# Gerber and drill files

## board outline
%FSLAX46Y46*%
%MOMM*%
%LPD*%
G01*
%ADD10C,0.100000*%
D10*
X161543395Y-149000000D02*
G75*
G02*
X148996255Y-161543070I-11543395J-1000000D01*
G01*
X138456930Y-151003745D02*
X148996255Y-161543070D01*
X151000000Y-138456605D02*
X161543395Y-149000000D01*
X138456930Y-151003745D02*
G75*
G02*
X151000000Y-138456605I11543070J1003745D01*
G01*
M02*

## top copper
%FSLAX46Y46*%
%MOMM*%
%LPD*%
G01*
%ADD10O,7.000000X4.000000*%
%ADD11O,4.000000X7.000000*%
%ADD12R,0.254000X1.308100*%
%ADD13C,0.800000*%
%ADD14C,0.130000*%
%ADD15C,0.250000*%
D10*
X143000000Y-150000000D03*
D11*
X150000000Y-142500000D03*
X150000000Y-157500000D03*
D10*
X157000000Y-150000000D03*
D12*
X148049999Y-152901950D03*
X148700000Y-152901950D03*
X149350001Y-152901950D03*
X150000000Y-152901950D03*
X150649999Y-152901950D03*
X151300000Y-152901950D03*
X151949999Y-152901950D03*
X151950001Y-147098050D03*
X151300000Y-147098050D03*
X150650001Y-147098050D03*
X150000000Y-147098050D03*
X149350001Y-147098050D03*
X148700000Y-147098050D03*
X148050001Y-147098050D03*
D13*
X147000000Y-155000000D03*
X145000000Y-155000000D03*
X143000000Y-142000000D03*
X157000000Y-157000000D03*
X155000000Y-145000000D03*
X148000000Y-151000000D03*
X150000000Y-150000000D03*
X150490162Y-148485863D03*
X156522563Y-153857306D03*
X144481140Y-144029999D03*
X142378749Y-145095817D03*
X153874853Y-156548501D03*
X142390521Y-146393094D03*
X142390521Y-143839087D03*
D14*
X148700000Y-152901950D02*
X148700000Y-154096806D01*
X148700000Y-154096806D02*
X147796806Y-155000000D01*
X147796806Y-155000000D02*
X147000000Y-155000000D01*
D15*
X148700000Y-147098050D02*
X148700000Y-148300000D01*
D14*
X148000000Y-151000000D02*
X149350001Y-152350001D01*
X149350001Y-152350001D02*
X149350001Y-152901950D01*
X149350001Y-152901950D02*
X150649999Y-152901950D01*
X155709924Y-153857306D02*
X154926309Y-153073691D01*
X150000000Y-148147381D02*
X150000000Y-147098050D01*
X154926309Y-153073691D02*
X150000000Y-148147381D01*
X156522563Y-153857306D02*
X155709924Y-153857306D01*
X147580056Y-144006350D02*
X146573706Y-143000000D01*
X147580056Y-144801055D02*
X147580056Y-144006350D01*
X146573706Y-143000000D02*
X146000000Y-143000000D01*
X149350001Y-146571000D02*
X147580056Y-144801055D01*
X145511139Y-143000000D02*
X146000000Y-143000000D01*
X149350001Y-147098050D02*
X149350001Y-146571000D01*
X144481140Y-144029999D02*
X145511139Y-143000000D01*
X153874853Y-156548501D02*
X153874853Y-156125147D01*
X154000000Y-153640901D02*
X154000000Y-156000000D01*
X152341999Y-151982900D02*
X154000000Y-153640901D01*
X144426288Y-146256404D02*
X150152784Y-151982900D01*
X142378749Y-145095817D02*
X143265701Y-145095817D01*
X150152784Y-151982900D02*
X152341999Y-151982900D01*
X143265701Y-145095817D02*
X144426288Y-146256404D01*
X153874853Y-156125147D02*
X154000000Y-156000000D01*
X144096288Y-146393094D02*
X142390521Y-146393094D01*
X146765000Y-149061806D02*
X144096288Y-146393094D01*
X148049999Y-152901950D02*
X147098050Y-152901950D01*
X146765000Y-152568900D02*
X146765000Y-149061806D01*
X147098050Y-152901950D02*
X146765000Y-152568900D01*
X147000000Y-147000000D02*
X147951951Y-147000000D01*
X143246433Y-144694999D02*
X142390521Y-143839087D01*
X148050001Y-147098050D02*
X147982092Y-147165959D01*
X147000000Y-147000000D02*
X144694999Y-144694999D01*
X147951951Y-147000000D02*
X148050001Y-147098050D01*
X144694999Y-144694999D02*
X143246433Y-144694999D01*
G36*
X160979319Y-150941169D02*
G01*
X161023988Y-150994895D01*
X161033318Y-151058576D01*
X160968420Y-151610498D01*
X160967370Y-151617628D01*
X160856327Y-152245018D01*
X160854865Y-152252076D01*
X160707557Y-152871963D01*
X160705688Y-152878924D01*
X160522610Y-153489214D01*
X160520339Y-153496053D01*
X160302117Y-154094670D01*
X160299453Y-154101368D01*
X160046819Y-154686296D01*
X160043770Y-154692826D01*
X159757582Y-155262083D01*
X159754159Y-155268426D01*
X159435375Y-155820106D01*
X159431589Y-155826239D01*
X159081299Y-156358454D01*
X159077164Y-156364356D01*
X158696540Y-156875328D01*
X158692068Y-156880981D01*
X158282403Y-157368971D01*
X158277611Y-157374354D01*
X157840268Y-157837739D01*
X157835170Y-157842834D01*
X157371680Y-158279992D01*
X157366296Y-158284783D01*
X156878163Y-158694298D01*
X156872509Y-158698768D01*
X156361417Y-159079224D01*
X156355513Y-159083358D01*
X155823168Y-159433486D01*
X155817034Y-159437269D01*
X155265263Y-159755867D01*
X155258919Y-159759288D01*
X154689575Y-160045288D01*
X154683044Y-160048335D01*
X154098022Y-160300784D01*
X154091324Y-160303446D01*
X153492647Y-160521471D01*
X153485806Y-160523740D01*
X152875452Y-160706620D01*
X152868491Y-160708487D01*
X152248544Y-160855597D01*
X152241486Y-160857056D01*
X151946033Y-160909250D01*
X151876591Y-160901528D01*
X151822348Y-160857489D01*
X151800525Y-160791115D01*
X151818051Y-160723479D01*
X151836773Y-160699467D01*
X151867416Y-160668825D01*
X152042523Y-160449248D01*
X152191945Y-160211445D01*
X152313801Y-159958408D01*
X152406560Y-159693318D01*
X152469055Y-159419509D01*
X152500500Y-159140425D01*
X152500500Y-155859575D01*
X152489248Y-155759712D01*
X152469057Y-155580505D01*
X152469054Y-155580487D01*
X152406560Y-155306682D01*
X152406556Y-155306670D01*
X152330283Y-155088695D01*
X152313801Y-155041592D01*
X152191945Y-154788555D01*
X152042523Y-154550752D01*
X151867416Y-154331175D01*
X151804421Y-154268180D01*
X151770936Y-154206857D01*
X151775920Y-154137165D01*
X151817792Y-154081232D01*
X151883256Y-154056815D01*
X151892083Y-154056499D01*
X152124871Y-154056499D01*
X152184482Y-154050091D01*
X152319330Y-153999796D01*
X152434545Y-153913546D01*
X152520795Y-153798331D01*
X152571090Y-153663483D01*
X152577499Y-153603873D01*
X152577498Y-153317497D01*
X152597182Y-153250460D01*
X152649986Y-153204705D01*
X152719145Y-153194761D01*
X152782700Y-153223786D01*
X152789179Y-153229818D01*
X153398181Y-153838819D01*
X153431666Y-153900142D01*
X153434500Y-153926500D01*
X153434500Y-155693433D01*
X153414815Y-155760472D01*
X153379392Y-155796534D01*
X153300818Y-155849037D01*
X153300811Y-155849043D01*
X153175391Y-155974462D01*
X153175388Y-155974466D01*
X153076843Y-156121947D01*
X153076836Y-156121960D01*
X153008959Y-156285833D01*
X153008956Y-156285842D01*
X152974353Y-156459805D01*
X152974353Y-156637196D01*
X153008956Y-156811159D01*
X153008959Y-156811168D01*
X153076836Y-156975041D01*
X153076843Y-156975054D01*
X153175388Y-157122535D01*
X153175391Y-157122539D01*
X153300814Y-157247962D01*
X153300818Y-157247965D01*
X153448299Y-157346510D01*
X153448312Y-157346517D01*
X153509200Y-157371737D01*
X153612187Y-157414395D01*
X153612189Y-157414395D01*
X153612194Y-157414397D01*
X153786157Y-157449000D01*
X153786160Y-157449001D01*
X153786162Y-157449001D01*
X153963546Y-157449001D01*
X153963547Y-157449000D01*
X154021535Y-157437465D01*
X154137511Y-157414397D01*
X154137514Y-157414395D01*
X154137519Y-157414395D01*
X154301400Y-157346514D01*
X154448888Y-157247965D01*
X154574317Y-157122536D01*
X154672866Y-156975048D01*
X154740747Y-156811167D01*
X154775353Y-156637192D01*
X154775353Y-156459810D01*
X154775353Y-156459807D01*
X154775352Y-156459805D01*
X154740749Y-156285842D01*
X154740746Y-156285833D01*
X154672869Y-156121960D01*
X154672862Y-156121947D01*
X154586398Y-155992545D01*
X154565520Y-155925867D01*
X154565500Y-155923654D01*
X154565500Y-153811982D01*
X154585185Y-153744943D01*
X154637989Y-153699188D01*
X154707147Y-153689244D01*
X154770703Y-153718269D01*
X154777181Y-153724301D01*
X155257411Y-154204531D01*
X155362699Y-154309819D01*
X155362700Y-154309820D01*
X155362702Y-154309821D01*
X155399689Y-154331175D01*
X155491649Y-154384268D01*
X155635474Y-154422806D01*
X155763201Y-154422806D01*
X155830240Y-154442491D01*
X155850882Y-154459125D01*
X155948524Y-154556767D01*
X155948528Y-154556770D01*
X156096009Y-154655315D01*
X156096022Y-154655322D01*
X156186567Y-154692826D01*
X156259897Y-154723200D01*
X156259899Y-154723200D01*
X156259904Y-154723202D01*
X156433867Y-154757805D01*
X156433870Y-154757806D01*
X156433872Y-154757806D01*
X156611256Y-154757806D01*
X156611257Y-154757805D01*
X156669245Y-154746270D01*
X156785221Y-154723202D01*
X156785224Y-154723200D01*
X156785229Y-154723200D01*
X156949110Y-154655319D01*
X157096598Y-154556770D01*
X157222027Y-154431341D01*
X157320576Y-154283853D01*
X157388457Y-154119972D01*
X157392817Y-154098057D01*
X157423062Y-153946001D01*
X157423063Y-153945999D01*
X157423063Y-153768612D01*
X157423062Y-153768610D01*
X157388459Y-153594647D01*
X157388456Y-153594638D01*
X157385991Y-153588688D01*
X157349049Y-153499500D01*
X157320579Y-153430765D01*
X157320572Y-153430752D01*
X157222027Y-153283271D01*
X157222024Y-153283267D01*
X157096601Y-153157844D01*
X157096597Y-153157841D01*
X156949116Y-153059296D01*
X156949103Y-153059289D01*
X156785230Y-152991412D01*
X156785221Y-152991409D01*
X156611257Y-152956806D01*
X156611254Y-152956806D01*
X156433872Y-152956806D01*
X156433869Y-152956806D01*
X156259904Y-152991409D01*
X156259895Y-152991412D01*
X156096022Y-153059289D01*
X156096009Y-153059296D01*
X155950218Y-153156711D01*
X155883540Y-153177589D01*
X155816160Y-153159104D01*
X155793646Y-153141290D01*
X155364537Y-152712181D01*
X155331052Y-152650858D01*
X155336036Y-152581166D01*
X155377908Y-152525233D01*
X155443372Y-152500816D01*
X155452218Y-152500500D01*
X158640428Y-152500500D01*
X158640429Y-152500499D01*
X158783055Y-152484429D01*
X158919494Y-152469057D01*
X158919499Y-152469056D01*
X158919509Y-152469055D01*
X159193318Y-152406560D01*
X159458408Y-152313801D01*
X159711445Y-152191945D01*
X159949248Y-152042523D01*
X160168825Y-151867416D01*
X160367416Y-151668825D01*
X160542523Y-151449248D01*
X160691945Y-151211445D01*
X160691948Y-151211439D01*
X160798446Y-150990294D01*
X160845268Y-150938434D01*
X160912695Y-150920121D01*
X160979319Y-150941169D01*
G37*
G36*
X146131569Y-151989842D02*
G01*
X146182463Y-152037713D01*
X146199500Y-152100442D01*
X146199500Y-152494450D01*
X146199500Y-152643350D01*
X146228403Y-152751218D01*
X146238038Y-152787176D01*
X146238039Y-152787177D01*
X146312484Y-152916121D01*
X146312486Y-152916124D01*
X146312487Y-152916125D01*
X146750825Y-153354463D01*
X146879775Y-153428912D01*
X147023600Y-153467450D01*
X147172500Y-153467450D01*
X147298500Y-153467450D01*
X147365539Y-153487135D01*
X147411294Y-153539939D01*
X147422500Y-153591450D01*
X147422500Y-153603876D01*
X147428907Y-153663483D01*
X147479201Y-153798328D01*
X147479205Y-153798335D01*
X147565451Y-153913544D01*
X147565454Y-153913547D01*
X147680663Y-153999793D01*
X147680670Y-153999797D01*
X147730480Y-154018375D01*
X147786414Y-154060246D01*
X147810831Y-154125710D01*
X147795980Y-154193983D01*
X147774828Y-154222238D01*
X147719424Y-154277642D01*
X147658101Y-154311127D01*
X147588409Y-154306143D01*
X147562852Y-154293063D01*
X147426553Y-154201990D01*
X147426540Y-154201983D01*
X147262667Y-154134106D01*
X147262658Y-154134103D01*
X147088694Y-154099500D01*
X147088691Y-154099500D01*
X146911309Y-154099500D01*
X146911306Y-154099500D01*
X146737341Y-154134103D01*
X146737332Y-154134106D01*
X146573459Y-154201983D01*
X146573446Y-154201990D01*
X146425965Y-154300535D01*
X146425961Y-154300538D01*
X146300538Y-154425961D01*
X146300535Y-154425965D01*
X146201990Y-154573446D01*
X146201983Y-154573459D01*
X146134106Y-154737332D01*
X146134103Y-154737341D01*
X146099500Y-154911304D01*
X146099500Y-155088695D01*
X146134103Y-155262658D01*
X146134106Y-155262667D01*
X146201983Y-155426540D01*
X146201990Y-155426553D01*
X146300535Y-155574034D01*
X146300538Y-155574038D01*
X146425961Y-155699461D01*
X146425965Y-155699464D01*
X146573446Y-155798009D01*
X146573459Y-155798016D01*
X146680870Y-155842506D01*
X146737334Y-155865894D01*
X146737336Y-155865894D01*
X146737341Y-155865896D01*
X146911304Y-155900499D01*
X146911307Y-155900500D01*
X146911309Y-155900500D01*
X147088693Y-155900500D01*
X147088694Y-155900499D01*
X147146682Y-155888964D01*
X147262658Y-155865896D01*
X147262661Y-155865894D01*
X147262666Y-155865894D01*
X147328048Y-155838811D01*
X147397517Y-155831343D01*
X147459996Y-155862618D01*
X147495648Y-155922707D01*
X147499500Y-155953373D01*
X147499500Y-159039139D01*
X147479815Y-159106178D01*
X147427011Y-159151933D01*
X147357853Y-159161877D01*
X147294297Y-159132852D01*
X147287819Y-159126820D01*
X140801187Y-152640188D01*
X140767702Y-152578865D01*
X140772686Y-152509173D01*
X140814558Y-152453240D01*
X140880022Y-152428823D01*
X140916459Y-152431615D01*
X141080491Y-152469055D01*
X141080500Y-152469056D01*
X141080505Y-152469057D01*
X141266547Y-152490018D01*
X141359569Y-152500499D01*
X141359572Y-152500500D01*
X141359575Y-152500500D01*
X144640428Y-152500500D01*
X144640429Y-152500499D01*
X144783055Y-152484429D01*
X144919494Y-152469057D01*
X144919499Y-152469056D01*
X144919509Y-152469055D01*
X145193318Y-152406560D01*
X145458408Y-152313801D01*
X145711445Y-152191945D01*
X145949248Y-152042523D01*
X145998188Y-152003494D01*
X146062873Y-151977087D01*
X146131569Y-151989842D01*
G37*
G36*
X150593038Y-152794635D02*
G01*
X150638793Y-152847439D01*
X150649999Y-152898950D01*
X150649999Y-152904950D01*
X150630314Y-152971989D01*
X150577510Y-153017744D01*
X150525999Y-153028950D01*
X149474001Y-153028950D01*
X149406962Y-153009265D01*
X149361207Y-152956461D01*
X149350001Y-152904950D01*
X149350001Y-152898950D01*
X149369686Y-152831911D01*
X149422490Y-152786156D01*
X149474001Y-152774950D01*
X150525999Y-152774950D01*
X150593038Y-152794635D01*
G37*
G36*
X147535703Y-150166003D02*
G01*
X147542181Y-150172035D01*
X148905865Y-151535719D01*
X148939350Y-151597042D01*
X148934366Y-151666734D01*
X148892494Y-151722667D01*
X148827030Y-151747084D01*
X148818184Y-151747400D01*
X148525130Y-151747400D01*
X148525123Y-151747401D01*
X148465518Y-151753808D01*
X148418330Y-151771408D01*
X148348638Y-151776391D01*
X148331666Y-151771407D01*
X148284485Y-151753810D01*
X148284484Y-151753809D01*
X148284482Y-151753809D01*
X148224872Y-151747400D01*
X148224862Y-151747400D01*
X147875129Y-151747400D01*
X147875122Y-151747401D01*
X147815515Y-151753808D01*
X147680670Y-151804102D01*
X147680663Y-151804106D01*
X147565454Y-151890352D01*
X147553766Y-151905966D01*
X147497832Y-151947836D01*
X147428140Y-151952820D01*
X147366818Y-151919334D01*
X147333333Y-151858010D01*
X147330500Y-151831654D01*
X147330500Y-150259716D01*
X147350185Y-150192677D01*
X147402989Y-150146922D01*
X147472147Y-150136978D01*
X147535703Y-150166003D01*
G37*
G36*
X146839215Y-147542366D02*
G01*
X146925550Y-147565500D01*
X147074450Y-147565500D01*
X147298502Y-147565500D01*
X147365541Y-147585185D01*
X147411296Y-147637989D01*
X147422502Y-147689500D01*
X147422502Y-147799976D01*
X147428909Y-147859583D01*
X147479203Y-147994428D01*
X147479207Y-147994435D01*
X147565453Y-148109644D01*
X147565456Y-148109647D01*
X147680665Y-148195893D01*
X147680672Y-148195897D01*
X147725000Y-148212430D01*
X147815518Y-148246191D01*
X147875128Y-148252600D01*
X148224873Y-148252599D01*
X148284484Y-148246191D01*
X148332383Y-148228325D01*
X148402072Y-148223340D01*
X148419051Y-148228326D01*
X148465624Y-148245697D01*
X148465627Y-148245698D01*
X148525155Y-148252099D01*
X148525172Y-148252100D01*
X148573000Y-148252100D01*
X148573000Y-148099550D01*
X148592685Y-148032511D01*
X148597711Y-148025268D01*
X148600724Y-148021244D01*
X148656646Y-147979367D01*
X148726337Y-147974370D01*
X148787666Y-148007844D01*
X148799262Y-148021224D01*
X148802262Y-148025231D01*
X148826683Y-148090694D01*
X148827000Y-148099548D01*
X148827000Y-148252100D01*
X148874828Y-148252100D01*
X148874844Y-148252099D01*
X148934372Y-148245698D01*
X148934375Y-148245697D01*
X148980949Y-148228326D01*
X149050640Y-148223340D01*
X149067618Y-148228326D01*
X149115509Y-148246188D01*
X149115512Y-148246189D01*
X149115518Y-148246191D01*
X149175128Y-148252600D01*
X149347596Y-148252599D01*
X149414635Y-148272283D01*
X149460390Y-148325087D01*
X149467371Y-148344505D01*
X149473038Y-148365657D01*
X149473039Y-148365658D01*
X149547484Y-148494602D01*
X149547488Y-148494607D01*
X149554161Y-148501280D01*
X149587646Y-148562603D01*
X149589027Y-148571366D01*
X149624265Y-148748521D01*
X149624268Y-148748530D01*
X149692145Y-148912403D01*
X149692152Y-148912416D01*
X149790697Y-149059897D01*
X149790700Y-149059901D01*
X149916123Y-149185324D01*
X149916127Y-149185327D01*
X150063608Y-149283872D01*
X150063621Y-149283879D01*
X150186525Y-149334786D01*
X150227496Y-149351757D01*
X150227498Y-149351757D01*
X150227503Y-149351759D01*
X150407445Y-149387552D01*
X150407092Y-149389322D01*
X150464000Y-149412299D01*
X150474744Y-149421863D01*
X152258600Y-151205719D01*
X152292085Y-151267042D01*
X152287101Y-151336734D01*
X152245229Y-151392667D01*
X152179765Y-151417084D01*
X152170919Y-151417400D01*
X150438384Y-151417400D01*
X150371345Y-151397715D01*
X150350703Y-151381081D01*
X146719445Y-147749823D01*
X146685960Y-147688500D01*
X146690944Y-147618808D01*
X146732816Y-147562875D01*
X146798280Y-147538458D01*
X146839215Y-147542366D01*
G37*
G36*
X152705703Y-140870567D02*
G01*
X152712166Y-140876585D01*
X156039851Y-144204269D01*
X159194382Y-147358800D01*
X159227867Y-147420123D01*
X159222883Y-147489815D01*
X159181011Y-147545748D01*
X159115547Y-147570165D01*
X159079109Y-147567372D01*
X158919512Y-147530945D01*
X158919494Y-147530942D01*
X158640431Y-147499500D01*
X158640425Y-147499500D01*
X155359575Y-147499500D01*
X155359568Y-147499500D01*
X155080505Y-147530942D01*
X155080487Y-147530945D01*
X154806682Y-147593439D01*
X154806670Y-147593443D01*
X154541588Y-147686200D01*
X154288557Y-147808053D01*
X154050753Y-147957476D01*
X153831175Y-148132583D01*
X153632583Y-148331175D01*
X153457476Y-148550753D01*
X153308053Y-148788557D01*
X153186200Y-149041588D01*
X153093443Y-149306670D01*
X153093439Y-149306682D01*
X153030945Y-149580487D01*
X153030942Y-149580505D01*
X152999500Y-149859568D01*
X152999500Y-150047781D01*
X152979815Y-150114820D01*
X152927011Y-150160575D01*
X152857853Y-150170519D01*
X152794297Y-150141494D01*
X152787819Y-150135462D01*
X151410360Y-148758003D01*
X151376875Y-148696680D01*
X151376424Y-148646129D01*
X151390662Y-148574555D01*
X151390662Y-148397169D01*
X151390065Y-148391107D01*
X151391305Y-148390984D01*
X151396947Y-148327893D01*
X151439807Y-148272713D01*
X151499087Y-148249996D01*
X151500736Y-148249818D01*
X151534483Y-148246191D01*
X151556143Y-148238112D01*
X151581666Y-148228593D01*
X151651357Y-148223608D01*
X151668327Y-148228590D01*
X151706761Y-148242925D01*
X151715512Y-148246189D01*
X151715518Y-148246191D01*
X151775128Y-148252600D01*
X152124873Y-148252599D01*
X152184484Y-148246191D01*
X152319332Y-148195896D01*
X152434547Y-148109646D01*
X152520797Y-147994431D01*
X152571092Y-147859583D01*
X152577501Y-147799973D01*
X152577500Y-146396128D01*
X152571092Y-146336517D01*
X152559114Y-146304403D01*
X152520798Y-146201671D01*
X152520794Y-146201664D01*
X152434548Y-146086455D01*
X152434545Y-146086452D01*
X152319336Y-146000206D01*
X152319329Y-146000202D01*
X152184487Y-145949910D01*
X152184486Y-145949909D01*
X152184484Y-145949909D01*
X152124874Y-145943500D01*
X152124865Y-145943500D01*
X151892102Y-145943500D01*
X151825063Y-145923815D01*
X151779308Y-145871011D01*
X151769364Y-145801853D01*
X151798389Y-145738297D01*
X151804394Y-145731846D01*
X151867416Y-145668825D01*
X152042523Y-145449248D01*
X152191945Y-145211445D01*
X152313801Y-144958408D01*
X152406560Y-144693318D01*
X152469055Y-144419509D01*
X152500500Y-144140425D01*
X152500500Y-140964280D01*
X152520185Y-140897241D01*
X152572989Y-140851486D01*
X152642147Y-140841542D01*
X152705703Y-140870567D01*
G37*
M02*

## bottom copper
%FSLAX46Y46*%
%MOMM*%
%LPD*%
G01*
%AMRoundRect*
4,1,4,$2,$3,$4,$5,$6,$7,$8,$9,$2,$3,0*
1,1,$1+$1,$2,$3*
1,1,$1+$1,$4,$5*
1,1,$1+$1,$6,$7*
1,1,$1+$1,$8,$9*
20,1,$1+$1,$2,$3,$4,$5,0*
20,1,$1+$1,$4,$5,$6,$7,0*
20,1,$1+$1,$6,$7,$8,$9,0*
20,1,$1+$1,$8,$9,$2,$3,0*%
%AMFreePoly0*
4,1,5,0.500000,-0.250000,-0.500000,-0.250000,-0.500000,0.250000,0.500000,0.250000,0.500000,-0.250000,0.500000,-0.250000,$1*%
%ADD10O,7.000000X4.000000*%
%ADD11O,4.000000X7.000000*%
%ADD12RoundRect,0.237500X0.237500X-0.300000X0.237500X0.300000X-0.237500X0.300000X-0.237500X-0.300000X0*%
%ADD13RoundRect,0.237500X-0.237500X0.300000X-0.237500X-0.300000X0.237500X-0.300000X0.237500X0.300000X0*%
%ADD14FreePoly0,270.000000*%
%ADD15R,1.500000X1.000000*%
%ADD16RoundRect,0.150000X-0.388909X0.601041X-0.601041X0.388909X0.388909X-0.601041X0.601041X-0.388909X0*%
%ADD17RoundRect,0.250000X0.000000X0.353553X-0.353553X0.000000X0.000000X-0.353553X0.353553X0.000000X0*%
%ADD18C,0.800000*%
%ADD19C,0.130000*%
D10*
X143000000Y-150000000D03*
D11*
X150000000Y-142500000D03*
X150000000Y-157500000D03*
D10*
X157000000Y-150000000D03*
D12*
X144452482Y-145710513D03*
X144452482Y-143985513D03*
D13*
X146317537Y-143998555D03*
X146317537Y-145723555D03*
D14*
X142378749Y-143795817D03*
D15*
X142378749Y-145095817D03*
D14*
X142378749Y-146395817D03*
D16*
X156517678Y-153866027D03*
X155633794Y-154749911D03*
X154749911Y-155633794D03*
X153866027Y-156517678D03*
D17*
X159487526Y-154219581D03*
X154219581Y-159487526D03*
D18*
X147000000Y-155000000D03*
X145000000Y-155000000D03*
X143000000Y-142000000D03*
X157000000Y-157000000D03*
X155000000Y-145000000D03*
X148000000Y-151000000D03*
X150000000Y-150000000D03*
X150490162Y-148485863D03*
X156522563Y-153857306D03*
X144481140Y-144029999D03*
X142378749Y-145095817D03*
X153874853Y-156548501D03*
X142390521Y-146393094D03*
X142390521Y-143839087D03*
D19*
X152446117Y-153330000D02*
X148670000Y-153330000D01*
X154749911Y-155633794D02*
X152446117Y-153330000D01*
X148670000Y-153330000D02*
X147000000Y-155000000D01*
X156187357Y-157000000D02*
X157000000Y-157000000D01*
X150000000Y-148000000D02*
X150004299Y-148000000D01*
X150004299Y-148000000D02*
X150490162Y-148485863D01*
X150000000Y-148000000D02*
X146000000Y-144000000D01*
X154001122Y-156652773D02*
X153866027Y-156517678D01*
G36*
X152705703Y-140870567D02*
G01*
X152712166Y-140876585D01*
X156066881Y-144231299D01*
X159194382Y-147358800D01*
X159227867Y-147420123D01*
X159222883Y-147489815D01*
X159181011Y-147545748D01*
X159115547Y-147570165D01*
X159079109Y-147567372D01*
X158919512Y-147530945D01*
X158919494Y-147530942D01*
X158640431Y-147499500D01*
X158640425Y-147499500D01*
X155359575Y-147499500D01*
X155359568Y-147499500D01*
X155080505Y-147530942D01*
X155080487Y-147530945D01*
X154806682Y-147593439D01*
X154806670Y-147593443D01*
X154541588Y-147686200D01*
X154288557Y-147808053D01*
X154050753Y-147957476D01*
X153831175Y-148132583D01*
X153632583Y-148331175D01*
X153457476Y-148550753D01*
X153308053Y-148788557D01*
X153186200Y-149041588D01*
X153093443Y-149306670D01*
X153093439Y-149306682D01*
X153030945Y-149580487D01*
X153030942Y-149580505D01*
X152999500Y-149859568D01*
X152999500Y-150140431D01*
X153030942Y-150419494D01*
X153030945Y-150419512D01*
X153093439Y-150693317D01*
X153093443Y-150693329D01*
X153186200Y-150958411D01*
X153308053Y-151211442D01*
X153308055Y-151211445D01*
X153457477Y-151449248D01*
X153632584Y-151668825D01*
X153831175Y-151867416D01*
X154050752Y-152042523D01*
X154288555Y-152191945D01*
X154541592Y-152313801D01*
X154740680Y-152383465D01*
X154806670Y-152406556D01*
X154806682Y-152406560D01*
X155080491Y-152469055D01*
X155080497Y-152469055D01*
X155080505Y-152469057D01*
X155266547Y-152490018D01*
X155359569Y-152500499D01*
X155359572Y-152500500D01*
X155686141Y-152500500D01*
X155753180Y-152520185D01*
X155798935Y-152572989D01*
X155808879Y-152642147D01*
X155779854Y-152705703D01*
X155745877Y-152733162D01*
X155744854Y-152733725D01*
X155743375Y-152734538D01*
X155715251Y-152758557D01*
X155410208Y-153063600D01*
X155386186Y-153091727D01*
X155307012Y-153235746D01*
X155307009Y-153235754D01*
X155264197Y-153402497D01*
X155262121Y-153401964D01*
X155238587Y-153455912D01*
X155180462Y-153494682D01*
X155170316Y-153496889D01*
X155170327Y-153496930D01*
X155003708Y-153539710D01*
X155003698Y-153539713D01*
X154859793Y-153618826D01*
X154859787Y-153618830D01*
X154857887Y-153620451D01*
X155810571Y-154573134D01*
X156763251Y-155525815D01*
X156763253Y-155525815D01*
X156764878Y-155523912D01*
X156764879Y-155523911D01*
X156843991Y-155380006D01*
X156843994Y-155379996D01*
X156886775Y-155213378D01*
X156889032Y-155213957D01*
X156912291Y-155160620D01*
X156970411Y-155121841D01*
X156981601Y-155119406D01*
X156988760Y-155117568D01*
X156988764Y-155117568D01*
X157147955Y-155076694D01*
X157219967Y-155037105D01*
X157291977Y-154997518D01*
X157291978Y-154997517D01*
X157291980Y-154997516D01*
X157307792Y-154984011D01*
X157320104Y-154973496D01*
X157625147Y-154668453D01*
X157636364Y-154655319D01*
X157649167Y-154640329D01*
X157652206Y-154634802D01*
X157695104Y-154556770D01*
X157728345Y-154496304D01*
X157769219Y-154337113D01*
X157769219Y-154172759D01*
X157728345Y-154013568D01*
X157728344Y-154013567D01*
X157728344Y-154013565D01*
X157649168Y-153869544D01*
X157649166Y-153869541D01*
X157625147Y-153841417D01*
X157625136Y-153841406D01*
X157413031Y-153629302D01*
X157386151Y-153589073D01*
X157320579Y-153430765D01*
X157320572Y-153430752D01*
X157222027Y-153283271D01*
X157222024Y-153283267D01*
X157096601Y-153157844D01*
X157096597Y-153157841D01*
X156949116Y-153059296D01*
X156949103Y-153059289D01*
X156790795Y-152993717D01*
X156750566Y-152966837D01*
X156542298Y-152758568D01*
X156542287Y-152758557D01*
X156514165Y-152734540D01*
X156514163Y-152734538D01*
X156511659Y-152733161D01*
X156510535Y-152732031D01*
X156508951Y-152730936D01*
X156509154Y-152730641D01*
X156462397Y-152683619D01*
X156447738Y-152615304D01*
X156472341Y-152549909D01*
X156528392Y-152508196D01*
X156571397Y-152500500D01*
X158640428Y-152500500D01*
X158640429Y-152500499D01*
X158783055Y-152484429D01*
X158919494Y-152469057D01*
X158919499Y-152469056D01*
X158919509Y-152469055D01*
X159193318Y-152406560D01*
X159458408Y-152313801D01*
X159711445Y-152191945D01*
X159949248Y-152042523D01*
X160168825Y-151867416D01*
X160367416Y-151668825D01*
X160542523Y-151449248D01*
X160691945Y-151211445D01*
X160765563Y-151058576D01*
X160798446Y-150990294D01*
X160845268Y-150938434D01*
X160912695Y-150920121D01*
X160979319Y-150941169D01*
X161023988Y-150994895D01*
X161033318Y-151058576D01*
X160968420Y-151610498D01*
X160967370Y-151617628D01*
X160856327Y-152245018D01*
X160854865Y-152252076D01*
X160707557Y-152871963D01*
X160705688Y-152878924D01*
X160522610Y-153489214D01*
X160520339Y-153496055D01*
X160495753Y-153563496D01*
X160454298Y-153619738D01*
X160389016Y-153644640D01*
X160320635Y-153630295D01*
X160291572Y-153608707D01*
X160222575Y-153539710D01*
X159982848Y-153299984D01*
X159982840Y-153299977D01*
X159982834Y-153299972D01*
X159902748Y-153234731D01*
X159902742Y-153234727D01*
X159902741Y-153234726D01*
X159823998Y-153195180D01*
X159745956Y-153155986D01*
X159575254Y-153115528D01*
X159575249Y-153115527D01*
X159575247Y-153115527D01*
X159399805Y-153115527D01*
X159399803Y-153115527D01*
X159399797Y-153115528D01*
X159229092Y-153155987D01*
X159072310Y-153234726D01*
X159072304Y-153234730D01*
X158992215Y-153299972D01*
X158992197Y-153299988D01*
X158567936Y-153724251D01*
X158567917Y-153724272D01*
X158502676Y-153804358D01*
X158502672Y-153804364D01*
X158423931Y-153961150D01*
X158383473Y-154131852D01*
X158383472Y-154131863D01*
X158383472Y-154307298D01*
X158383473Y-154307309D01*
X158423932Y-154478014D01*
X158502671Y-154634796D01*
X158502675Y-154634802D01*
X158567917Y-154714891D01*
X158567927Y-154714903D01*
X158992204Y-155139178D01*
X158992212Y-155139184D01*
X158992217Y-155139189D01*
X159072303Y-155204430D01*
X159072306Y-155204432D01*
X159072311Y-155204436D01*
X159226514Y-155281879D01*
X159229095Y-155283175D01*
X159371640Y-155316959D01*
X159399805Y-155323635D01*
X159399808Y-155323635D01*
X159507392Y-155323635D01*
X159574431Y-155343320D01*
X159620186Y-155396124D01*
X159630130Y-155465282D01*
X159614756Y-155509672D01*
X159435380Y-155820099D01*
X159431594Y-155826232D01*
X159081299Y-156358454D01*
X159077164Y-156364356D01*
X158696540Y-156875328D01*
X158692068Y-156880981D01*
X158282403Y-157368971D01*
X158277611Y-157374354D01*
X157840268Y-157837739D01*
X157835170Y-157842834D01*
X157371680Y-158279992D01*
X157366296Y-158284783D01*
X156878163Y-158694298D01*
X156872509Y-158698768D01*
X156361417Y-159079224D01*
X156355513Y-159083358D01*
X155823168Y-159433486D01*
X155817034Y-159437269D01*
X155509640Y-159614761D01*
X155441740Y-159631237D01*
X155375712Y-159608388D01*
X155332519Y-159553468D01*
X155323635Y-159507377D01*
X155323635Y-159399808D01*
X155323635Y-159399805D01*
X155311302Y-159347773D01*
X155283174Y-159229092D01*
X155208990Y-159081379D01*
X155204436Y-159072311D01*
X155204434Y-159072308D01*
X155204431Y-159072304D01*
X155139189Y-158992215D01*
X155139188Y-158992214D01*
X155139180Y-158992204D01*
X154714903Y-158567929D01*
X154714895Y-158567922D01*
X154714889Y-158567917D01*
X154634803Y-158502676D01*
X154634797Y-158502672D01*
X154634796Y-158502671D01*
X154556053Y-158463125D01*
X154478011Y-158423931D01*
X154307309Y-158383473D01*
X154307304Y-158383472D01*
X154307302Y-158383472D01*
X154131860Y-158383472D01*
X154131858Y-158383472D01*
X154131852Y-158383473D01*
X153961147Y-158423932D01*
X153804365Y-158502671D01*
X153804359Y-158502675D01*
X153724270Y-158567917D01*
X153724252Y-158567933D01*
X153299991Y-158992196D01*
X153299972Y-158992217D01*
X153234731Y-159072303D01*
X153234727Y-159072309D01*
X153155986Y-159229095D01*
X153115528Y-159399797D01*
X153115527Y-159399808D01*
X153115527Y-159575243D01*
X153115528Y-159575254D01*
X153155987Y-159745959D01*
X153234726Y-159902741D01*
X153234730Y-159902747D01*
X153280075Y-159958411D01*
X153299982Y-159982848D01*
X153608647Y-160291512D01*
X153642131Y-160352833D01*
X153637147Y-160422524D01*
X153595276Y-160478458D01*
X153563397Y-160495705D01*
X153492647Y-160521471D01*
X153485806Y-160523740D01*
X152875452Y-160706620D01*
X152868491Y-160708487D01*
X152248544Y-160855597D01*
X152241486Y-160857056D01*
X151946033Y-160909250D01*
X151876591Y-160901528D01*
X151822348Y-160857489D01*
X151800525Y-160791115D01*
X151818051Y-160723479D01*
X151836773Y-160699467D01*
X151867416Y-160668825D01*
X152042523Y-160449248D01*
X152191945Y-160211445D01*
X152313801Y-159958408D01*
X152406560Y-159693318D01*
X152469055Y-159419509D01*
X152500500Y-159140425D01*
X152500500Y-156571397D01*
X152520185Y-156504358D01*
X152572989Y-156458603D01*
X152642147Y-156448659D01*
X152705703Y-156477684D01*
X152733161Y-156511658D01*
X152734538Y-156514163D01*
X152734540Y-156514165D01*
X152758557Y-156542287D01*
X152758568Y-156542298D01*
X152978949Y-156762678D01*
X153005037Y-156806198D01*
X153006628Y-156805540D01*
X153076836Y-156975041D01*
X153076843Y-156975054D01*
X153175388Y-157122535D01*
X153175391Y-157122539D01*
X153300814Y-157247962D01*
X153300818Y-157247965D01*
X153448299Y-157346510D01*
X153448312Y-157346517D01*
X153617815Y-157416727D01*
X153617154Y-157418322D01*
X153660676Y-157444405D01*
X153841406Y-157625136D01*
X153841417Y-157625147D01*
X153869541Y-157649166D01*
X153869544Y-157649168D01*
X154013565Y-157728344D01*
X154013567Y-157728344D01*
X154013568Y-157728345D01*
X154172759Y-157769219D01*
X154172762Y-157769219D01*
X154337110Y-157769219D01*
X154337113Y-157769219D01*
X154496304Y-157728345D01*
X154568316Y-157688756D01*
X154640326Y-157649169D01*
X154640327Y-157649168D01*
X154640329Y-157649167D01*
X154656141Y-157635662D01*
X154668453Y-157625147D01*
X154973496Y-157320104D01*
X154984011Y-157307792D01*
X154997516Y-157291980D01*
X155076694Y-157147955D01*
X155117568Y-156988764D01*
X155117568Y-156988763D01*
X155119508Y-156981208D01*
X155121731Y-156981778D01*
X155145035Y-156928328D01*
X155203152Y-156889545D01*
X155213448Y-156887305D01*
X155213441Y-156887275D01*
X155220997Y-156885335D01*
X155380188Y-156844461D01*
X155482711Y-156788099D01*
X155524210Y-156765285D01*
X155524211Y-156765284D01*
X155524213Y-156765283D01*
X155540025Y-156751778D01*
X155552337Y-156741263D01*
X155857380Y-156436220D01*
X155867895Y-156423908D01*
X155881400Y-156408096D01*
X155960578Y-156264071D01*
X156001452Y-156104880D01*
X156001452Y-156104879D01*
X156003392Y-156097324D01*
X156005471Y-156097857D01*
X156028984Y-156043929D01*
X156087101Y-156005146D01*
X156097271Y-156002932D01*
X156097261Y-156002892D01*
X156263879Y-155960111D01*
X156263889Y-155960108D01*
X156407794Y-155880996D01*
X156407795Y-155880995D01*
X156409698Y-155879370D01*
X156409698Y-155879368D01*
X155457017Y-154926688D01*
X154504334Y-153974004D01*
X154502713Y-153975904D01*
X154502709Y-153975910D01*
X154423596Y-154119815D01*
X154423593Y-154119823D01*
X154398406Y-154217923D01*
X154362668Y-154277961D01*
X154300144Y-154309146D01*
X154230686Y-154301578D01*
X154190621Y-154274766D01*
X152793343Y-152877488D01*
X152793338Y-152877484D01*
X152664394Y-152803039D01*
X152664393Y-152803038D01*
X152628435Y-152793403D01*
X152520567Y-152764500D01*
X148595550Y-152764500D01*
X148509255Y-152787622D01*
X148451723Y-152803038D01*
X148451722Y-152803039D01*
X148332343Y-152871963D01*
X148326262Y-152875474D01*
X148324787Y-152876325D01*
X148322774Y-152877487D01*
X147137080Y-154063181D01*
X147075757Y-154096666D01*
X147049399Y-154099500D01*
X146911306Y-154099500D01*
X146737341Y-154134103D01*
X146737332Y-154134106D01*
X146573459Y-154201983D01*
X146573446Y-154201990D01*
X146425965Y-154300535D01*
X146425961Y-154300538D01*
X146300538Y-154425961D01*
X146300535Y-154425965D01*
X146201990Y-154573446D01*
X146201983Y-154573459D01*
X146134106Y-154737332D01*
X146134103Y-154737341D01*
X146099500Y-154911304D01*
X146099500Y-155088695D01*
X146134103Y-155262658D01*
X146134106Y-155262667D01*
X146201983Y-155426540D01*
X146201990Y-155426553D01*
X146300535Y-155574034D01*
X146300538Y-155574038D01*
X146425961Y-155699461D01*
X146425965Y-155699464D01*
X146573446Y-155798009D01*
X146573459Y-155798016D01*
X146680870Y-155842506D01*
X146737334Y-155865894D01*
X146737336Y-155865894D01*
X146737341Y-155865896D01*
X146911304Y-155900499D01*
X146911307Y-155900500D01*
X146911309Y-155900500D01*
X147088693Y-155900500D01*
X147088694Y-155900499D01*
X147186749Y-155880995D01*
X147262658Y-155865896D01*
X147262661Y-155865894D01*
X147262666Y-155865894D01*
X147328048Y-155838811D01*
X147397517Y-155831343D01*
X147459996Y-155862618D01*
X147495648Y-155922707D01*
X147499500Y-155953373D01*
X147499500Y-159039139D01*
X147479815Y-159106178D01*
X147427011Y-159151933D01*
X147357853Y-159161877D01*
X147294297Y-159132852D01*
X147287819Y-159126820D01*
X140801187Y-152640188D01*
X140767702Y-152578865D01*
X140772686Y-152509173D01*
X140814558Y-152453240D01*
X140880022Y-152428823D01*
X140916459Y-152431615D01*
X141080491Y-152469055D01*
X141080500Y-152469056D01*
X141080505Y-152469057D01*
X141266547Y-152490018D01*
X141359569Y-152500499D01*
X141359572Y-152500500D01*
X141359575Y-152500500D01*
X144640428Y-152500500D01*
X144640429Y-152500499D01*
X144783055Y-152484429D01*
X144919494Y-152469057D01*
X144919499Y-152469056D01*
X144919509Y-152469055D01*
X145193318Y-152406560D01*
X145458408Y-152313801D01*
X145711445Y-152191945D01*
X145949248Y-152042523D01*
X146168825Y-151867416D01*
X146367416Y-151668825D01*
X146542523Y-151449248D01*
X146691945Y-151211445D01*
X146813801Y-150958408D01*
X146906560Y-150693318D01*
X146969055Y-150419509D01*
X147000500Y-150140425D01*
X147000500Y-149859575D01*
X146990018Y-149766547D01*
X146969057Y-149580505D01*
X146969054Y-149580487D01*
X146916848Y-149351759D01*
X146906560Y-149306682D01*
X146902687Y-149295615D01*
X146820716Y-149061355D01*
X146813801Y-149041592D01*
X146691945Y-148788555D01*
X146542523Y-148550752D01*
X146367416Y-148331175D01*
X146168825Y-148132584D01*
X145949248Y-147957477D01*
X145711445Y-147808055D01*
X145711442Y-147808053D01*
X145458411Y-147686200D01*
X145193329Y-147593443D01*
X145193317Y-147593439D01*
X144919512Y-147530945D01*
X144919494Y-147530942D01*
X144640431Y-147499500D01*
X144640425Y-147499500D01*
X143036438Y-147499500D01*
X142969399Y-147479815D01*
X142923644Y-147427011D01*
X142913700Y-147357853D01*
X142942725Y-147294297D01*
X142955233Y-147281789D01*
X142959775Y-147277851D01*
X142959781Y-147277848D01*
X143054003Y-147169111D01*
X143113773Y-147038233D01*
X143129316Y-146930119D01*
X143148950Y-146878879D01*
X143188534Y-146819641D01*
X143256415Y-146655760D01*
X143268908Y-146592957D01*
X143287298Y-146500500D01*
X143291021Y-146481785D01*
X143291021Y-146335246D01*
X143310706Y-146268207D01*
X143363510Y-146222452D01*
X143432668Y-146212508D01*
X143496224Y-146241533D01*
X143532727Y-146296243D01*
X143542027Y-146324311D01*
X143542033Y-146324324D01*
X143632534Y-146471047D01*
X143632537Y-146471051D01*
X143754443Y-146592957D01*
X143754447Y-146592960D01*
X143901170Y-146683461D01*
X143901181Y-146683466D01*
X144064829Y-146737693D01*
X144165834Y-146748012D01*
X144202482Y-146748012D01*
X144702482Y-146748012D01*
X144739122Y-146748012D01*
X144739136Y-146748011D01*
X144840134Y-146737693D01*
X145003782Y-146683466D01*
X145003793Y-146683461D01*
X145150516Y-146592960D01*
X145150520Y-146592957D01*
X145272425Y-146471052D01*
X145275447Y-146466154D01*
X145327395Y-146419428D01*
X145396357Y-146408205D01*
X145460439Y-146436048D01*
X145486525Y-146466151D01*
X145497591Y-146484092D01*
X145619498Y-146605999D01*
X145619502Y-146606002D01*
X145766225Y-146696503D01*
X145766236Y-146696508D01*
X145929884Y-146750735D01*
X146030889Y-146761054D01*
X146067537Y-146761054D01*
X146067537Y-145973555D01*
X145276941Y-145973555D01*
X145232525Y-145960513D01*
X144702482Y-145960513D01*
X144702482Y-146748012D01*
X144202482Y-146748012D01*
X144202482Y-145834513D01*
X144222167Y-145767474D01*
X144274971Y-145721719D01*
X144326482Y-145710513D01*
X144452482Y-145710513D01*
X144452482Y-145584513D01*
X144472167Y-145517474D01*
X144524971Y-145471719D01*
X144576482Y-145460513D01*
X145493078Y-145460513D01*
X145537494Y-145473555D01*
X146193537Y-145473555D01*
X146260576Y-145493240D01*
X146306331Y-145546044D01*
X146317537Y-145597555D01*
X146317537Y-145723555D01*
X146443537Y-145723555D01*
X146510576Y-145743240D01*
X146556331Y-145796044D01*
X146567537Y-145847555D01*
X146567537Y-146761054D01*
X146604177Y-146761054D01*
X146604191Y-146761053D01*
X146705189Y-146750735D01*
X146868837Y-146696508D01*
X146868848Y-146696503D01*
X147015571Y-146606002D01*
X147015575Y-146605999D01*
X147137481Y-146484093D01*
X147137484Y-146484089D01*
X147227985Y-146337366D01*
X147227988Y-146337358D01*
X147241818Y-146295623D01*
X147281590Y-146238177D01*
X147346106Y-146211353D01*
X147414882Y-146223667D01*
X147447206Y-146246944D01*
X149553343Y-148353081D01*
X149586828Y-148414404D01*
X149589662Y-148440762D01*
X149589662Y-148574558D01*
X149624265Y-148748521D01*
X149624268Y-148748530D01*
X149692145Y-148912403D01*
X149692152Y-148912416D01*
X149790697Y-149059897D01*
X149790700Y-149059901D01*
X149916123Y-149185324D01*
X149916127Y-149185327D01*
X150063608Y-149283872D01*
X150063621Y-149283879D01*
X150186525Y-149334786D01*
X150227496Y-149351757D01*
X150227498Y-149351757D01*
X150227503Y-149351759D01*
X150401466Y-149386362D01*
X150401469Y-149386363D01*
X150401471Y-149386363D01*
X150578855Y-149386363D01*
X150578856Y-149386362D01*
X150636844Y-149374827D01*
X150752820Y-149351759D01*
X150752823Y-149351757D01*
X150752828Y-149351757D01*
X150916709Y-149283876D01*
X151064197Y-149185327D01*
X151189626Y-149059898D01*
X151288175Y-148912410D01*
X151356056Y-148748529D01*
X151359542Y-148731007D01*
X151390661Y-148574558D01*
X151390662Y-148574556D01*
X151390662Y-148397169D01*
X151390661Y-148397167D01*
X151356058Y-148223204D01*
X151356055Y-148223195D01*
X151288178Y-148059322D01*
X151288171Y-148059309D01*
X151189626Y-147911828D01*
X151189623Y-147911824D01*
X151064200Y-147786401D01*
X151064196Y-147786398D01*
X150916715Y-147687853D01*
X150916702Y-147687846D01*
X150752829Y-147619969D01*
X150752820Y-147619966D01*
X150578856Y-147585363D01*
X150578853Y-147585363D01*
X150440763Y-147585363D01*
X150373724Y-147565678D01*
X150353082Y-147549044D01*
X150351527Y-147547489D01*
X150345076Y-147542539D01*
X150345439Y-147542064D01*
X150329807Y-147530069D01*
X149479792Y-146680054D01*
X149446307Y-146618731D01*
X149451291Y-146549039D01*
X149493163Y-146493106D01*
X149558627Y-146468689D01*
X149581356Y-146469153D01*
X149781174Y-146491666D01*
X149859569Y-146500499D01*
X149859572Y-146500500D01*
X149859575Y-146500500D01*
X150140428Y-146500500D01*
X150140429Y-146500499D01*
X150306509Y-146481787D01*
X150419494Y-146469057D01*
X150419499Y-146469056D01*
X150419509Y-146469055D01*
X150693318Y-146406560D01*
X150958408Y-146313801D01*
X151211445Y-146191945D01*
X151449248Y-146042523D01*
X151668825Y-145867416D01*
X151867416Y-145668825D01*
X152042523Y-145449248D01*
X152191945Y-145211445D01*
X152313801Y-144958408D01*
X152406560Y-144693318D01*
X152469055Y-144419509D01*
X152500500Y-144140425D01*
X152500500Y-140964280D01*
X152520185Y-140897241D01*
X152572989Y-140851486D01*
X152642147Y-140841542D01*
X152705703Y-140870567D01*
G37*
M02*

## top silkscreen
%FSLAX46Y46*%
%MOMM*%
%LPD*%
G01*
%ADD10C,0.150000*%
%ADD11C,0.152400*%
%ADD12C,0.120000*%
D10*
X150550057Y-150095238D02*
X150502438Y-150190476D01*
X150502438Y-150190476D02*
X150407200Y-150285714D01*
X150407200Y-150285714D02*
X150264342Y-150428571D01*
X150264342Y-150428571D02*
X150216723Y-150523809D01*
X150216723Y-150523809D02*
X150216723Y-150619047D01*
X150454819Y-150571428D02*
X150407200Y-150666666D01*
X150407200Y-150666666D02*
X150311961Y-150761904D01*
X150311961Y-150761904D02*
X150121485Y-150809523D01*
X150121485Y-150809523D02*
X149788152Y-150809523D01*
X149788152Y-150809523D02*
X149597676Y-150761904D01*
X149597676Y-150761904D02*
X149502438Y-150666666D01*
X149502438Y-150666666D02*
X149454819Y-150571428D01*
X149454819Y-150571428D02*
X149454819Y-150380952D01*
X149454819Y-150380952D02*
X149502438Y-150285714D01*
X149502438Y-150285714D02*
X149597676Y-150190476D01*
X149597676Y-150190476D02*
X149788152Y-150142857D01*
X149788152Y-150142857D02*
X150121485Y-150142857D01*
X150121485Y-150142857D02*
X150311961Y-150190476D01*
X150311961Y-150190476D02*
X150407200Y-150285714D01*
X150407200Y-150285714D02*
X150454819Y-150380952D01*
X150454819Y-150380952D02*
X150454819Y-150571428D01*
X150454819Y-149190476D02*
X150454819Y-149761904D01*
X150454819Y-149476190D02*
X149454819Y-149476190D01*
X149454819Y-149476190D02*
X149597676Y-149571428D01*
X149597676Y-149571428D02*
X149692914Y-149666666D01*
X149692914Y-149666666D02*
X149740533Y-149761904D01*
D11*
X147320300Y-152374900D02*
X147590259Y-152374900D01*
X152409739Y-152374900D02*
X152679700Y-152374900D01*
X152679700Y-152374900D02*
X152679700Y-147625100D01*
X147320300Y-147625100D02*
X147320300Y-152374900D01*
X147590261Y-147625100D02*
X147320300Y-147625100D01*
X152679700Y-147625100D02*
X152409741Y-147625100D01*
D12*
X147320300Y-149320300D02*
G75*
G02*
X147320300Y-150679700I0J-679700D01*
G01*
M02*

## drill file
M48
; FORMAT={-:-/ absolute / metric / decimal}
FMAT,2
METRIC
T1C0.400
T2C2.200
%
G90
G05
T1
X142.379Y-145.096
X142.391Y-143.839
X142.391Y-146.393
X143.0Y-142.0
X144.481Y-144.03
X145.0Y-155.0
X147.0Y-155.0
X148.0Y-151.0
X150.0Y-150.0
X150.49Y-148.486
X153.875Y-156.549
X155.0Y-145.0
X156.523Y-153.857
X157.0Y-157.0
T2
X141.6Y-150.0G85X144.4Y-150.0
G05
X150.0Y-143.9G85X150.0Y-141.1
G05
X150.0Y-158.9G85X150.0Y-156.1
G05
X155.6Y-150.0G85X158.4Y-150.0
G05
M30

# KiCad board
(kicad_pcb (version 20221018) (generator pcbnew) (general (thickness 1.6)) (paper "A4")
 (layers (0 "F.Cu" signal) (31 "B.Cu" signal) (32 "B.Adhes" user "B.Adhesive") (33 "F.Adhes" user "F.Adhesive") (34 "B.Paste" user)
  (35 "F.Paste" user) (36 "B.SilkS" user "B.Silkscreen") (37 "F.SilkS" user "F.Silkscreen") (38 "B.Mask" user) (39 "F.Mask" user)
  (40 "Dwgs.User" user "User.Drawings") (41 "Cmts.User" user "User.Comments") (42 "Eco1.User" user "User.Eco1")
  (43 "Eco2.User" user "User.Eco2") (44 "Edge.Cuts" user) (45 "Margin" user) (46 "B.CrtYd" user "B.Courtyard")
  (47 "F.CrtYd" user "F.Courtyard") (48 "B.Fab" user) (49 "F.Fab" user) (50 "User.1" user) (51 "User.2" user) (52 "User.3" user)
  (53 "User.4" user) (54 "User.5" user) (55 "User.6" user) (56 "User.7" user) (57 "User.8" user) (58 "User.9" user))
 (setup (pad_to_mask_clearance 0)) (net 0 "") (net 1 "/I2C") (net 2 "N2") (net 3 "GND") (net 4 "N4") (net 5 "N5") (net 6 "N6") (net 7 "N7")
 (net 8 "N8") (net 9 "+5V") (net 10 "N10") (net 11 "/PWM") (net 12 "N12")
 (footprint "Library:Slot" (layer "F.Cu") (at 150 150)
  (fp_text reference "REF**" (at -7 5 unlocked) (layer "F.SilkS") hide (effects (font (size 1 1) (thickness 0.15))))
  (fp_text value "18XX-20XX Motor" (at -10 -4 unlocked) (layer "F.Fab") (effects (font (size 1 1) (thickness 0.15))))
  (pad "1" thru_hole oval (at -7 0 90) (size 4 7) (drill oval 2.2 5) (layers "*.Cu" "*.Mask"))
  (pad "1" thru_hole oval (at 0 -7.5 180) (size 4 7) (drill oval 2.2 5) (layers "*.Cu" "*.Mask"))
  (pad "1" thru_hole oval (at 0 7.5 180) (size 4 7) (drill oval 2.2 5) (layers "*.Cu" "*.Mask"))
  (pad "1" thru_hole oval (at 7 0 90) (size 4 7) (drill oval 2.2 5) (layers "*.Cu" "*.Mask")))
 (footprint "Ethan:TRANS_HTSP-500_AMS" (layer "F.Cu") (at 150 150 90)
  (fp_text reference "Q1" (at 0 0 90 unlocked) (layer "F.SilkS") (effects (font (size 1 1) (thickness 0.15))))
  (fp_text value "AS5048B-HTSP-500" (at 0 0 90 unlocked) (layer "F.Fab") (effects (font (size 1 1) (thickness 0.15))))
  (fp_line (start -2.3749 -2.6797) (end -2.3749 -2.409741) (stroke (width 0.1524) (type solid)) (layer "F.SilkS"))
  (fp_line (start -2.3749 2.409739) (end -2.3749 2.6797) (stroke (width 0.1524) (type solid)) (layer "F.SilkS"))
  (fp_line (start -2.3749 2.6797) (end 2.3749 2.6797) (stroke (width 0.1524) (type solid)) (layer "F.SilkS"))
  (fp_line (start 2.3749 -2.6797) (end -2.3749 -2.6797) (stroke (width 0.1524) (type solid)) (layer "F.SilkS"))
  (fp_line (start 2.3749 -2.409739) (end 2.3749 -2.6797) (stroke (width 0.1524) (type solid)) (layer "F.SilkS"))
  (fp_line (start 2.3749 2.6797) (end 2.3749 2.409741) (stroke (width 0.1524) (type solid)) (layer "F.SilkS"))
  (fp_arc (start 0.6797 -2.6797) (mid 0 -2) (end -0.6797 -2.6797) (stroke (width 0.12) (type default)) (layer "F.SilkS"))
  (pad "1" smd rect (at -2.90195 -1.950001 90) (size 1.3081 0.254) (layers "F.Cu" "F.Paste" "F.Mask") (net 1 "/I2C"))
  (pad "2" smd rect (at -2.90195 -1.3 90) (size 1.3081 0.254) (layers "F.Cu" "F.Paste" "F.Mask") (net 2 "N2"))
  (pad "3" smd rect (at -2.90195 -0.649999 90) (size 1.3081 0.254) (layers "F.Cu" "F.Paste" "F.Mask") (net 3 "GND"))
  (pad "4" smd rect (at -2.90195 0 90) (size 1.3081 0.254) (layers "F.Cu" "F.Paste" "F.Mask") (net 3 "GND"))
  (pad "5" smd rect (at -2.90195 0.649999 90) (size 1.3081 0.254) (layers "F.Cu" "F.Paste" "F.Mask") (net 3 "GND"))
  (pad "6" smd rect (at -2.90195 1.3 90) (size 1.3081 0.254) (layers "F.Cu" "F.Paste" "F.Mask") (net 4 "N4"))
  (pad "7" smd rect (at -2.90195 1.949999 90) (size 1.3081 0.254) (layers "F.Cu" "F.Paste" "F.Mask") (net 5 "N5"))
  (pad "8" smd rect (at 2.90195 1.950001 90) (size 1.3081 0.254) (layers "F.Cu" "F.Paste" "F.Mask") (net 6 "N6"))
  (pad "9" smd rect (at 2.90195 1.3 90) (size 1.3081 0.254) (layers "F.Cu" "F.Paste" "F.Mask") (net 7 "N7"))
  (pad "10" smd rect (at 2.90195 0.650001 90) (size 1.3081 0.254) (layers "F.Cu" "F.Paste" "F.Mask") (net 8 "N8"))
  (pad "11" smd rect (at 2.90195 0 90) (size 1.3081 0.254) (layers "F.Cu" "F.Paste" "F.Mask") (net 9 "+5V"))
  (pad "12" smd rect (at 2.90195 -0.649999 90) (size 1.3081 0.254) (layers "F.Cu" "F.Paste" "F.Mask") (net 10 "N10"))
  (pad "13" smd rect (at 2.90195 -1.3 90) (size 1.3081 0.254) (layers "F.Cu" "F.Paste" "F.Mask") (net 3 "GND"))
  (pad "14" smd rect (at 2.90195 -1.949999 90) (size 1.3081 0.254) (layers "F.Cu" "F.Paste" "F.Mask") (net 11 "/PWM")))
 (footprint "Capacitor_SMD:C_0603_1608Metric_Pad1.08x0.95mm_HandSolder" (layer "B.Cu") (at 144.452482 144.848013 90)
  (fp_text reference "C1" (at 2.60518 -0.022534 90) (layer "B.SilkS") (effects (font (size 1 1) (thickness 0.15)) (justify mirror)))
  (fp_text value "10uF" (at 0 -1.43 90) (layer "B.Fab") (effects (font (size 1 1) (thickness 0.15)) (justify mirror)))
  (pad "1" smd roundrect (at -0.8625 0 90) (size 1.075 0.95) (layers "B.Cu" "B.Paste" "B.Mask") (roundrect_rratio 0.25) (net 3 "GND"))
  (pad "2" smd roundrect (at 0.8625 0 90) (size 1.075 0.95) (layers "B.Cu" "B.Paste" "B.Mask") (roundrect_rratio 0.25) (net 10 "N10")))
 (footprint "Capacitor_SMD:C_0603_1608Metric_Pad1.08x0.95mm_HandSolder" (layer "B.Cu") (at 146.317537 144.861055 -90)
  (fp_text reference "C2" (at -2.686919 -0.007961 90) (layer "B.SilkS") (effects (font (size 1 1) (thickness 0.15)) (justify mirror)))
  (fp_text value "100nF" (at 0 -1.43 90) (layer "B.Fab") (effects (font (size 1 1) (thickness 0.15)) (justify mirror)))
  (pad "1" smd roundrect (at -0.8625 0 270) (size 1.075 0.95) (layers "B.Cu" "B.Paste" "B.Mask") (roundrect_rratio 0.25) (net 9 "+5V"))
  (pad "2" smd roundrect (at 0.8625 0 270) (size 1.075 0.95) (layers "B.Cu" "B.Paste" "B.Mask") (roundrect_rratio 0.25) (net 3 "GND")))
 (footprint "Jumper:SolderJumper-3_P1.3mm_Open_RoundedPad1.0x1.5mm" (layer "B.Cu") (at 142.378749 145.095817 -90)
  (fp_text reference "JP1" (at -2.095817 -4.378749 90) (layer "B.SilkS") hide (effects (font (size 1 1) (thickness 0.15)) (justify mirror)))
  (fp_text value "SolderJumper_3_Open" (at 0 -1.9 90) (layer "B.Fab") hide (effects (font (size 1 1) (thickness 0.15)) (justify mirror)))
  (pad "1" smd custom (at -1.3 0 270) (size 1 0.5) (layers "B.Cu" "B.Mask") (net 11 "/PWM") (zone_connect 2)
   (options (clearance outline) (anchor rect)) (primitives))
  (pad "2" smd rect (at 0 0 270) (size 1 1.5) (layers "B.Cu" "B.Mask") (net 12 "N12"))
  (pad "3" smd custom (at 1.3 0 270) (size 1 0.5) (layers "B.Cu" "B.Mask") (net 1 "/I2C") (zone_connect 2)
   (options (clearance outline) (anchor rect)) (primitives)))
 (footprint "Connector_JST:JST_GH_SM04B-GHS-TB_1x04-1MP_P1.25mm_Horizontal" (layer "B.Cu") (at 156.5 156.5 -135)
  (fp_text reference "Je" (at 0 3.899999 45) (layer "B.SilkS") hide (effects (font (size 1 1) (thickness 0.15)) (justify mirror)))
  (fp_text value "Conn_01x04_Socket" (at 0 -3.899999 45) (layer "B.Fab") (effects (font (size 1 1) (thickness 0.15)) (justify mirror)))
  (pad "1" smd roundrect (at -1.875 1.85 225) (size 0.6 1.7) (layers "B.Cu" "B.Paste" "B.Mask") (roundrect_rratio 0.25) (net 9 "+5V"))
  (pad "2" smd roundrect (at -0.625 1.85 225) (size 0.6 1.7) (layers "B.Cu" "B.Paste" "B.Mask") (roundrect_rratio 0.25) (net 3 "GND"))
  (pad "3" smd roundrect (at 0.625 1.85 225) (size 0.6 1.7) (layers "B.Cu" "B.Paste" "B.Mask") (roundrect_rratio 0.25) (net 2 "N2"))
  (pad "4" smd roundrect (at 1.875 1.85 225) (size 0.6 1.7) (layers "B.Cu" "B.Paste" "B.Mask") (roundrect_rratio 0.25) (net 12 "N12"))
  (pad "MP" smd roundrect (at -3.725 -0.5 225) (size 1 1) (layers "B.Cu" "B.Paste" "B.Mask") (roundrect_rratio 0.25))
  (pad "MP" smd roundrect (at 3.725 -0.5 225) (size 1 1) (layers "B.Cu" "B.Paste" "B.Mask") (roundrect_rratio 0.25)))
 (gr_arc (start 161.543395 149) (mid 158.191655 158.194313) (end 148.996255 161.54307) (stroke (width 0.1) (type default))
  (layer "Edge.Cuts"))
 (gr_line (start 138.45693 151.003745) (end 148.996255 161.54307) (stroke (width 0.1) (type default)) (layer "Edge.Cuts"))
 (gr_line (start 151 138.456605) (end 161.543395 149) (stroke (width 0.1) (type default)) (layer "Edge.Cuts"))
 (gr_arc (start 138.45693 151.003745) (mid 141.805687 141.808345) (end 151 138.456605) (stroke (width 0.1) (type default))
  (layer "Edge.Cuts"))
 (segment (start 148.7 152.90195) (end 148.7 154.096806) (width 0.13) (layer "F.Cu") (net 2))
 (segment (start 148.7 154.096806) (end 147.796806 155) (width 0.13) (layer "F.Cu") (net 2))
 (segment (start 147.796806 155) (end 147 155) (width 0.13) (layer "F.Cu") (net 2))
 (via (at 147 155) (size 0.8) (drill 0.4) (layers "F.Cu" "B.Cu") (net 2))
 (segment (start 152.446117 153.33) (end 148.67 153.33) (width 0.13) (layer "B.Cu") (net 2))
 (segment (start 154.749911 155.633794) (end 152.446117 153.33) (width 0.13) (layer "B.Cu") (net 2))
 (segment (start 148.67 153.33) (end 147 155) (width 0.13) (layer "B.Cu") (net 2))
 (segment (start 148.7 147.09805) (end 148.7 148.3) (width 0.25) (layer "F.Cu") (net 3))
 (segment (start 148 151) (end 149.350001 152.350001) (width 0.13) (layer "F.Cu") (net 3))
 (segment (start 149.350001 152.350001) (end 149.350001 152.90195) (width 0.13) (layer "F.Cu") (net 3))
 (segment (start 149.350001 152.90195) (end 150.649999 152.90195) (width 0.13) (layer "F.Cu") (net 3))
 (via (at 145 155) (size 0.8) (drill 0.4) (layers "F.Cu" "B.Cu") (free) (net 3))
 (via (at 143 142) (size 0.8) (drill 0.4) (layers "F.Cu" "B.Cu") (free) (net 3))
 (via (at 157 157) (size 0.8) (drill 0.4) (layers "F.Cu" "B.Cu") (free) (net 3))
 (via (at 155 145) (size 0.8) (drill 0.4) (layers "F.Cu" "B.Cu") (free) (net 3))
 (via (at 148 151) (size 0.8) (drill 0.4) (layers "F.Cu" "B.Cu") (free) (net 3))
 (via (at 150 150) (size 0.8) (drill 0.4) (layers "F.Cu" "B.Cu") (free) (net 3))
 (segment (start 156.187357 157) (end 157 157) (width 0.13) (layer "B.Cu") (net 3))
 (segment (start 155.709924 153.857306) (end 154.926309 153.073691) (width 0.13) (layer "F.Cu") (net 9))
 (segment (start 150 148.147381) (end 150 147.09805) (width 0.13) (layer "F.Cu") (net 9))
 (segment (start 154.926309 153.073691) (end 150 148.147381) (width 0.13) (layer "F.Cu") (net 9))
 (segment (start 156.522563 153.857306) (end 155.709924 153.857306) (width 0.13) (layer "F.Cu") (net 9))
 (via (at 150.490162 148.485863) (size 0.8) (drill 0.4) (layers "F.Cu" "B.Cu") (free) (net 9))
 (via (at 156.522563 153.857306) (size 0.8) (drill 0.4) (layers "F.Cu" "B.Cu") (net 9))
 (segment (start 150 148) (end 150.004299 148) (width 0.13) (layer "B.Cu") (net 9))
 (segment (start 150.004299 148) (end 150.490162 148.485863) (width 0.13) (layer "B.Cu") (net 9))
 (segment (start 150 148) (end 146 144) (width 0.13) (layer "B.Cu") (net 9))
 (segment (start 147.580056 144.00635) (end 146.573706 143) (width 0.13) (layer "F.Cu") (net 10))
 (segment (start 147.580056 144.801055) (end 147.580056 144.00635) (width 0.13) (layer "F.Cu") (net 10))
 (segment (start 146.573706 143) (end 146 143) (width 0.13) (layer "F.Cu") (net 10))
 (segment (start 149.350001 146.571) (end 147.580056 144.801055) (width 0.13) (layer "F.Cu") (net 10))
 (segment (start 145.511139 143) (end 146 143) (width 0.13) (layer "F.Cu") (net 10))
 (segment (start 149.350001 147.09805) (end 149.350001 146.571) (width 0.13) (layer "F.Cu") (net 10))
 (segment (start 144.48114 144.029999) (end 145.511139 143) (width 0.13) (layer "F.Cu") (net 10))
 (via (at 144.48114 144.029999) (size 0.8) (drill 0.4) (layers "F.Cu" "B.Cu") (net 10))
 (segment (start 153.874853 156.548501) (end 153.874853 156.125147) (width 0.13) (layer "F.Cu") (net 12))
 (segment (start 154 153.640901) (end 154 156) (width 0.13) (layer "F.Cu") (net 12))
 (segment (start 152.341999 151.9829) (end 154 153.640901) (width 0.13) (layer "F.Cu") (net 12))
 (segment (start 144.426288 146.256404) (end 150.152784 151.9829) (width 0.13) (layer "F.Cu") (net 12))
 (segment (start 142.378749 145.095817) (end 143.265701 145.095817) (width 0.13) (layer "F.Cu") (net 12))
 (segment (start 150.152784 151.9829) (end 152.341999 151.9829) (width 0.13) (layer "F.Cu") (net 12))
 (segment (start 143.265701 145.095817) (end 144.426288 146.256404) (width 0.13) (layer "F.Cu") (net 12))
 (segment (start 153.874853 156.125147) (end 154 156) (width 0.13) (layer "F.Cu") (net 12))
 (via (at 142.378749 145.095817) (size 0.8) (drill 0.4) (layers "F.Cu" "B.Cu") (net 12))
 (via (at 153.874853 156.548501) (size 0.8) (drill 0.4) (layers "F.Cu" "B.Cu") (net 12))
 (segment (start 154.001122 156.652773) (end 153.866027 156.517678) (width 0.13) (layer "B.Cu") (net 12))
 (segment (start 144.096288 146.393094) (end 142.390521 146.393094) (width 0.13) (layer "F.Cu") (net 1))
 (segment (start 146.765 149.061806) (end 144.096288 146.393094) (width 0.13) (layer "F.Cu") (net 1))
 (segment (start 148.049999 152.90195) (end 147.09805 152.90195) (width 0.13) (layer "F.Cu") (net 1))
 (segment (start 146.765 152.5689) (end 146.765 149.061806) (width 0.13) (layer "F.Cu") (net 1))
 (segment (start 147.09805 152.90195) (end 146.765 152.5689) (width 0.13) (layer "F.Cu") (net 1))
 (via (at 142.390521 146.393094) (size 0.8) (drill 0.4) (layers "F.Cu" "B.Cu") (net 1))
 (segment (start 147 147) (end 147.951951 147) (width 0.13) (layer "F.Cu") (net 11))
 (segment (start 143.246433 144.694999) (end 142.390521 143.839087) (width 0.13) (layer "F.Cu") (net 11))
 (segment (start 148.050001 147.09805) (end 147.982092 147.165959) (width 0.13) (layer "F.Cu") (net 11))
 (segment (start 147 147) (end 144.694999 144.694999) (width 0.13) (layer "F.Cu") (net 11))
 (segment (start 147.951951 147) (end 148.050001 147.09805) (width 0.13) (layer "F.Cu") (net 11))
 (segment (start 144.694999 144.694999) (end 143.246433 144.694999) (width 0.13) (layer "F.Cu") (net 11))
 (via (at 142.390521 143.839087) (size 0.8) (drill 0.4) (layers "F.Cu" "B.Cu") (free) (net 11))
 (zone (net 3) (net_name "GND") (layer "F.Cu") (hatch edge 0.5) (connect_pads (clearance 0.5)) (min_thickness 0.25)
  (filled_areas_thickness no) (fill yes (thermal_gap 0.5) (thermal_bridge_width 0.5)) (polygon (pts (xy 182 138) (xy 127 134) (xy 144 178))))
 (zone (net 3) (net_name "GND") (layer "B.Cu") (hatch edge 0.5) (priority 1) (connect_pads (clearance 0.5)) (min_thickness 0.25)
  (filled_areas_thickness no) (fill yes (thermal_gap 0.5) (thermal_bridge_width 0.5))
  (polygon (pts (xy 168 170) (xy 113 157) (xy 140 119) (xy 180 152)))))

